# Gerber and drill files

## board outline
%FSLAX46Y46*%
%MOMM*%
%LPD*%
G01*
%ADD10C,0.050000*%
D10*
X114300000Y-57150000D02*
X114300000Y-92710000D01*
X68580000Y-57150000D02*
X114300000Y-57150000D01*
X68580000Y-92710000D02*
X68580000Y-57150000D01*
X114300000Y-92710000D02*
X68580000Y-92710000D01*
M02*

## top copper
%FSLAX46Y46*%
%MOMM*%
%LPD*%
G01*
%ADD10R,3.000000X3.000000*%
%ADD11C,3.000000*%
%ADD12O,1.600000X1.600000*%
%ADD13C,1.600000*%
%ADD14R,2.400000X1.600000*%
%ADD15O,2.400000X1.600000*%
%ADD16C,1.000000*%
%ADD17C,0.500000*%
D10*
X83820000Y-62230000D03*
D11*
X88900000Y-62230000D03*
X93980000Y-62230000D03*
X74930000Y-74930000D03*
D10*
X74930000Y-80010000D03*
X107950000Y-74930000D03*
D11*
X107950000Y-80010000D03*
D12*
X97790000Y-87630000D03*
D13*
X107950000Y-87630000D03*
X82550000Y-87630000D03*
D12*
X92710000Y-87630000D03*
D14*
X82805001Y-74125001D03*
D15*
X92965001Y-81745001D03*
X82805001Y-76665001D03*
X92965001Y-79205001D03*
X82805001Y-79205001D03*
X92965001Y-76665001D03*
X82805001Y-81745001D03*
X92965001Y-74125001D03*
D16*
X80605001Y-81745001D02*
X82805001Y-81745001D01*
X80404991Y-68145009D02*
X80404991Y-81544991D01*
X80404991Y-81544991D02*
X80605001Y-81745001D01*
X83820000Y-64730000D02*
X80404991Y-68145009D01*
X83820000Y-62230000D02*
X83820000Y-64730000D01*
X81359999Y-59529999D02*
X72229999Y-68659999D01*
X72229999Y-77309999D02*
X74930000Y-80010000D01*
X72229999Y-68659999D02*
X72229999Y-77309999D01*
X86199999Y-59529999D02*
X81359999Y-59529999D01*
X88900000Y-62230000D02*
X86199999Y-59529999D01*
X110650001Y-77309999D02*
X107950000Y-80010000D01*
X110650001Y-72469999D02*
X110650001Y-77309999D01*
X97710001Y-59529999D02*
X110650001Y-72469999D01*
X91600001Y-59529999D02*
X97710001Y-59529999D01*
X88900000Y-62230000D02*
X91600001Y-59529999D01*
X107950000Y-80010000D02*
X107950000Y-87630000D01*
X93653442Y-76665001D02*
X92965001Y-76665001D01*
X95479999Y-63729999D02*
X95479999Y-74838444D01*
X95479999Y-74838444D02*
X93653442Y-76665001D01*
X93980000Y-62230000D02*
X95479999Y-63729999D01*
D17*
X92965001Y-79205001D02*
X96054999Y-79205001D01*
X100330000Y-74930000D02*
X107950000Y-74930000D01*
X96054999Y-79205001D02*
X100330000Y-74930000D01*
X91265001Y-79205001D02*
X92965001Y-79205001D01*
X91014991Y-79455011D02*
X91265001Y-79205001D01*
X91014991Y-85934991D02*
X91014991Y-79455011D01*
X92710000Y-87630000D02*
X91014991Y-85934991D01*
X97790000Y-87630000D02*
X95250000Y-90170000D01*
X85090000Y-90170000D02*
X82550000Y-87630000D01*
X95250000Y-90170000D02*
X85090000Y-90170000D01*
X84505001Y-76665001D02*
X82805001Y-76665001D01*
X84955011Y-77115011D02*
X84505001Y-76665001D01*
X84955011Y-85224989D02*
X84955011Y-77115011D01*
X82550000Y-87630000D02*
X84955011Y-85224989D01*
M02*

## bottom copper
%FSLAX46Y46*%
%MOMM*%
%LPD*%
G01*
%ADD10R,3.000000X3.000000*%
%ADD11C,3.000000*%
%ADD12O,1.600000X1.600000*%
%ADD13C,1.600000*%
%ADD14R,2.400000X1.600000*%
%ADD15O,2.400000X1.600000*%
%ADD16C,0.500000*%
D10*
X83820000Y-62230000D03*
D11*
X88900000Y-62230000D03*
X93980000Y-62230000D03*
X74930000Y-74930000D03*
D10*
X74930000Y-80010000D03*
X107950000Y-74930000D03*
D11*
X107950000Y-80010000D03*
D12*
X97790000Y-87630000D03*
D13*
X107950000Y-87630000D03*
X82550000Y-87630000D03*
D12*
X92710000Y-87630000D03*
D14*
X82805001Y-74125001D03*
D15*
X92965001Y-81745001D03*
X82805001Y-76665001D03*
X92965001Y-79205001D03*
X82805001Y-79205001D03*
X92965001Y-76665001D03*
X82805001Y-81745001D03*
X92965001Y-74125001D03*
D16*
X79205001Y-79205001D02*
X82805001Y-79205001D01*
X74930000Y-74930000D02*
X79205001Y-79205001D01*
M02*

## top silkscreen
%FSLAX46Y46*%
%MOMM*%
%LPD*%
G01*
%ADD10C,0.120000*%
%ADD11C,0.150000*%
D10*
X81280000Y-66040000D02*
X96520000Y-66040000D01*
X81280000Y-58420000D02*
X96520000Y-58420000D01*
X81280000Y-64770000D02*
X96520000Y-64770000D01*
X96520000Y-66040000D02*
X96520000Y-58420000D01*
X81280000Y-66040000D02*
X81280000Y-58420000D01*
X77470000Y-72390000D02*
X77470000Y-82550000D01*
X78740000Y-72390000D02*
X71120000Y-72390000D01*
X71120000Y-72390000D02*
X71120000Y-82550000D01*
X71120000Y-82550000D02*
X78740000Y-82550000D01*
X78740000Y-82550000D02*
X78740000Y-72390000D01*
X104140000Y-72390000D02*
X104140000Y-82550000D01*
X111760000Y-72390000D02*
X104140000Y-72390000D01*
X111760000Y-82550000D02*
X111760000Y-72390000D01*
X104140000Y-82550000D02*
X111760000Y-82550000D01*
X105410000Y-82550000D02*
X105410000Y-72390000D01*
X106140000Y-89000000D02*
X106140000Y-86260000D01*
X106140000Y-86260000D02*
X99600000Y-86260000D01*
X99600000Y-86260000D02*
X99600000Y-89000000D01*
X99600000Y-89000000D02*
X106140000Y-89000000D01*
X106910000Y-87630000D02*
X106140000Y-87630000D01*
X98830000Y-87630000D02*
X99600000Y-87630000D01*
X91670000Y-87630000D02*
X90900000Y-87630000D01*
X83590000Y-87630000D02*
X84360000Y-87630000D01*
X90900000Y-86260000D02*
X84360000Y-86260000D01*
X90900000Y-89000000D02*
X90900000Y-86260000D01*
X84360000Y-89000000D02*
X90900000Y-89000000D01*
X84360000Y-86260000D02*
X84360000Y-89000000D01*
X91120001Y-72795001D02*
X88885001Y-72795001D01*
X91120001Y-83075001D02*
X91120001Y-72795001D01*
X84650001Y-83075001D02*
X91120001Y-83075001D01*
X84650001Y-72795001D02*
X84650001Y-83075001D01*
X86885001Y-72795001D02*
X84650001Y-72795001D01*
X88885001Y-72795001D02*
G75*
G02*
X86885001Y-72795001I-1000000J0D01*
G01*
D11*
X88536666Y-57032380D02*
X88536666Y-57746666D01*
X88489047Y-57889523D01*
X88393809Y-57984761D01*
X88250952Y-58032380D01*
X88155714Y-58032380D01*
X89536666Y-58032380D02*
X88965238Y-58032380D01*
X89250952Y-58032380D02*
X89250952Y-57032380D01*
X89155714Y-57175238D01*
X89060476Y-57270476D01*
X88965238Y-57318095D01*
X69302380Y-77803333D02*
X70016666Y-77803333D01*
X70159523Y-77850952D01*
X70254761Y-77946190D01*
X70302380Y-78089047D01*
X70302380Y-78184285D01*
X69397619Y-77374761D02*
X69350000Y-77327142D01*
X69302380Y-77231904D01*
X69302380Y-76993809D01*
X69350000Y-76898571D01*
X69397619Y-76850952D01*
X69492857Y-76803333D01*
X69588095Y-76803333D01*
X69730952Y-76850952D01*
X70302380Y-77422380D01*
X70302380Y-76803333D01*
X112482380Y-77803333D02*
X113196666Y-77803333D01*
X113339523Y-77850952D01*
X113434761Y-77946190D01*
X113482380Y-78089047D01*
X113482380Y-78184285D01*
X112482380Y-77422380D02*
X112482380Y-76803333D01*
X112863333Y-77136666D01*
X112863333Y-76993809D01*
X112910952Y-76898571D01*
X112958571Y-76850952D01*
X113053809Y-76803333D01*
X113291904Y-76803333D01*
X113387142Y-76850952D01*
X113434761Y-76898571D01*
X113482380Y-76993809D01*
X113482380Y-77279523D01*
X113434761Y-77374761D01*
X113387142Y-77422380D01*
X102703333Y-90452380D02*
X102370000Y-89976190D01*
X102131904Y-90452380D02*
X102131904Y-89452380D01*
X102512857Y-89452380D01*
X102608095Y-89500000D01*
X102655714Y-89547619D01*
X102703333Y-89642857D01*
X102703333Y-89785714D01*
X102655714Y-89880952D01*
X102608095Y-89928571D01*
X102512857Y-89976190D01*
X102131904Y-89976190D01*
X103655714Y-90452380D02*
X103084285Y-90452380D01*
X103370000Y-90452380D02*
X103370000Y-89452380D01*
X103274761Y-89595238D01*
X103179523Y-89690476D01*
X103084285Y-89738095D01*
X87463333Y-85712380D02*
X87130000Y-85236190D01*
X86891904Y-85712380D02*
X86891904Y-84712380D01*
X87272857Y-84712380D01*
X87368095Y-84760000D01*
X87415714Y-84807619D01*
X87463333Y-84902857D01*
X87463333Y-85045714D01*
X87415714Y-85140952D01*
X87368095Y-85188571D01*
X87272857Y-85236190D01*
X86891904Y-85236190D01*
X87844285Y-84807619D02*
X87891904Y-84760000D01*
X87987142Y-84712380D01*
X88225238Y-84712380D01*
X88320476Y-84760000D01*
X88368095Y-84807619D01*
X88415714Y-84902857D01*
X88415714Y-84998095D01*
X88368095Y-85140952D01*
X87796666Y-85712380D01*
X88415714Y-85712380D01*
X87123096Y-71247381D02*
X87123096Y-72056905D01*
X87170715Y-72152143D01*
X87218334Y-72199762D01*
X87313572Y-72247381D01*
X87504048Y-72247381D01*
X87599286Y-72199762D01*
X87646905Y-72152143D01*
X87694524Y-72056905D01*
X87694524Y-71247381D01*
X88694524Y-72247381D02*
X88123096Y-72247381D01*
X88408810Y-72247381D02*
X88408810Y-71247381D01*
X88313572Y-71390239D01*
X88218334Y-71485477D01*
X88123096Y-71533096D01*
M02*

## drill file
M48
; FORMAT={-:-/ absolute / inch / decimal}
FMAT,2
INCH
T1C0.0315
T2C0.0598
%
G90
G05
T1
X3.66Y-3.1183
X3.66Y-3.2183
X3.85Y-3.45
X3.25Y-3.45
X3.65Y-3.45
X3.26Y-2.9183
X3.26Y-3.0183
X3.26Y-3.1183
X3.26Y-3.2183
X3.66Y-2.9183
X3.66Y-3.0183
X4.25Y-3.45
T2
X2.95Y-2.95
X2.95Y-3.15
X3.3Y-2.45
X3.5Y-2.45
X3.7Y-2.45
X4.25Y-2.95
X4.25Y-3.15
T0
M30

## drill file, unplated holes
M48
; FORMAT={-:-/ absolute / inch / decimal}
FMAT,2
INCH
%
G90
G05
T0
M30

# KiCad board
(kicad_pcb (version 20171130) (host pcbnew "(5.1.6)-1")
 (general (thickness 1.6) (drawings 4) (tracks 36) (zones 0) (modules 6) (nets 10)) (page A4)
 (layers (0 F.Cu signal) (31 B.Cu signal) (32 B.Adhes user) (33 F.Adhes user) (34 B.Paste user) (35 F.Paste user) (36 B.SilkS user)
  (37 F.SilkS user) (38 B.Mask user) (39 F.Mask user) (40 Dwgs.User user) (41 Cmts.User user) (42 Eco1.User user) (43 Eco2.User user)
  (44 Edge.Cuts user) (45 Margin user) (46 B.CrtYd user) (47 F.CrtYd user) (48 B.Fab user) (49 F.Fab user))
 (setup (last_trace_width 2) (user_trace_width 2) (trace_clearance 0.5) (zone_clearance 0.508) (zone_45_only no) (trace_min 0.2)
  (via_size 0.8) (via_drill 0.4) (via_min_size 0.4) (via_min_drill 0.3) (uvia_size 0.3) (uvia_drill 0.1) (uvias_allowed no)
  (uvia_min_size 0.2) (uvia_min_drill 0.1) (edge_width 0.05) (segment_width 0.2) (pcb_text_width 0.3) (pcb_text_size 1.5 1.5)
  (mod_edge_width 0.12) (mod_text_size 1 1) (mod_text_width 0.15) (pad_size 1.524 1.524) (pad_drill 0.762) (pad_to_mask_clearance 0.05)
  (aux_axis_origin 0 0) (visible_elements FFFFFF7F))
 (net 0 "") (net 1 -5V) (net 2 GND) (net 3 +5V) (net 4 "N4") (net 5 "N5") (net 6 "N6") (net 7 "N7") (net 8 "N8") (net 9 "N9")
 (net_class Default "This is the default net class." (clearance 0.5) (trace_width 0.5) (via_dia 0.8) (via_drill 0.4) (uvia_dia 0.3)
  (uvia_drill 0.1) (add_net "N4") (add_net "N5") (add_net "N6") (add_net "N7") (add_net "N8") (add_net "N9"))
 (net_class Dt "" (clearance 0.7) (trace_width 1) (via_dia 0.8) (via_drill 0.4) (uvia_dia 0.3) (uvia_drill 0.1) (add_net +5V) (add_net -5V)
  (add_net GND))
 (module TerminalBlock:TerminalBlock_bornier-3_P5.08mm (layer F.Cu) (at 83.82 62.23)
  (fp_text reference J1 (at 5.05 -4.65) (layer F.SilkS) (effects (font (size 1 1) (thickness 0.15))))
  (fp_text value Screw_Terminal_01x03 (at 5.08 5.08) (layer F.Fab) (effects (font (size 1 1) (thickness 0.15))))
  (fp_line (start -2.54 3.81) (end 12.7 3.81) (layer F.SilkS) (width 0.12))
  (fp_line (start -2.54 -3.81) (end 12.7 -3.81) (layer F.SilkS) (width 0.12))
  (fp_line (start -2.54 2.54) (end 12.7 2.54) (layer F.SilkS) (width 0.12))
  (fp_line (start 12.7 3.81) (end 12.7 -3.81) (layer F.SilkS) (width 0.12))
  (fp_line (start -2.54 3.81) (end -2.54 -3.81) (layer F.SilkS) (width 0.12))
  (pad 1 thru_hole rect (at 0 0) (size 3 3) (drill 1.52) (layers *.Cu *.Mask) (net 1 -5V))
  (pad 2 thru_hole circle (at 5.08 0) (size 3 3) (drill 1.52) (layers *.Cu *.Mask) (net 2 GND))
  (pad 3 thru_hole circle (at 10.16 0) (size 3 3) (drill 1.52) (layers *.Cu *.Mask) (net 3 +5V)))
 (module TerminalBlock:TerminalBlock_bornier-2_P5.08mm (layer F.Cu) (at 74.93 80.01 90)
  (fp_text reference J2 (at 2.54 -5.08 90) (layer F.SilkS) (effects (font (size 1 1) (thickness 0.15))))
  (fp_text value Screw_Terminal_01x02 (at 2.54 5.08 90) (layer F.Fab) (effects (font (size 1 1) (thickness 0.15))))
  (fp_line (start 7.62 2.54) (end -2.54 2.54) (layer F.SilkS) (width 0.12))
  (fp_line (start 7.62 3.81) (end 7.62 -3.81) (layer F.SilkS) (width 0.12))
  (fp_line (start 7.62 -3.81) (end -2.54 -3.81) (layer F.SilkS) (width 0.12))
  (fp_line (start -2.54 -3.81) (end -2.54 3.81) (layer F.SilkS) (width 0.12))
  (fp_line (start -2.54 3.81) (end 7.62 3.81) (layer F.SilkS) (width 0.12))
  (pad 2 thru_hole circle (at 5.08 0 90) (size 3 3) (drill 1.52) (layers *.Cu *.Mask) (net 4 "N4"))
  (pad 1 thru_hole rect (at 0 0 90) (size 3 3) (drill 1.52) (layers *.Cu *.Mask) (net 2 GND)))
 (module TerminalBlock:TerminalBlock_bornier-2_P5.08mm (layer F.Cu) (at 107.95 74.93 270)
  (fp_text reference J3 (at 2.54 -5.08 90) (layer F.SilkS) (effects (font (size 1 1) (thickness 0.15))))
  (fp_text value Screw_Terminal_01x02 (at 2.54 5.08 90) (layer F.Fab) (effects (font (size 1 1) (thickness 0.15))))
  (fp_line (start -2.54 3.81) (end 7.62 3.81) (layer F.SilkS) (width 0.12))
  (fp_line (start -2.54 -3.81) (end -2.54 3.81) (layer F.SilkS) (width 0.12))
  (fp_line (start 7.62 -3.81) (end -2.54 -3.81) (layer F.SilkS) (width 0.12))
  (fp_line (start 7.62 3.81) (end 7.62 -3.81) (layer F.SilkS) (width 0.12))
  (fp_line (start 7.62 2.54) (end -2.54 2.54) (layer F.SilkS) (width 0.12))
  (pad 1 thru_hole rect (at 0 0 270) (size 3 3) (drill 1.52) (layers *.Cu *.Mask) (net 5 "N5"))
  (pad 2 thru_hole circle (at 5.08 0 270) (size 3 3) (drill 1.52) (layers *.Cu *.Mask) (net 2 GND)))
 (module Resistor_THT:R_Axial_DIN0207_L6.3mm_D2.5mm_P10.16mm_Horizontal (layer F.Cu) (at 107.95 87.63 180)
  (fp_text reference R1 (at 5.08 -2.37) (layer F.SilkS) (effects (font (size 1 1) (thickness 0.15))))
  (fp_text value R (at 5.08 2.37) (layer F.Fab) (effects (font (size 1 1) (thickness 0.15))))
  (fp_line (start 1.81 -1.37) (end 1.81 1.37) (layer F.SilkS) (width 0.12))
  (fp_line (start 1.81 1.37) (end 8.35 1.37) (layer F.SilkS) (width 0.12))
  (fp_line (start 8.35 1.37) (end 8.35 -1.37) (layer F.SilkS) (width 0.12))
  (fp_line (start 8.35 -1.37) (end 1.81 -1.37) (layer F.SilkS) (width 0.12))
  (fp_line (start 1.04 0) (end 1.81 0) (layer F.SilkS) (width 0.12))
  (fp_line (start 9.12 0) (end 8.35 0) (layer F.SilkS) (width 0.12))
  (pad 2 thru_hole oval (at 10.16 0 180) (size 1.6 1.6) (drill 0.8) (layers *.Cu *.Mask) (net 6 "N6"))
  (pad 1 thru_hole circle (at 0 0 180) (size 1.6 1.6) (drill 0.8) (layers *.Cu *.Mask) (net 2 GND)))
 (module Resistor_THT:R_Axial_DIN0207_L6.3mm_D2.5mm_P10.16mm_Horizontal (layer F.Cu) (at 82.55 87.63)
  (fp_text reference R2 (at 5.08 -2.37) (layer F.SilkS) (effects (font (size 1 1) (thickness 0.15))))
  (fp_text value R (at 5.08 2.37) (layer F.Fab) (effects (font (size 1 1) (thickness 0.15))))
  (fp_line (start 9.12 0) (end 8.35 0) (layer F.SilkS) (width 0.12))
  (fp_line (start 1.04 0) (end 1.81 0) (layer F.SilkS) (width 0.12))
  (fp_line (start 8.35 -1.37) (end 1.81 -1.37) (layer F.SilkS) (width 0.12))
  (fp_line (start 8.35 1.37) (end 8.35 -1.37) (layer F.SilkS) (width 0.12))
  (fp_line (start 1.81 1.37) (end 8.35 1.37) (layer F.SilkS) (width 0.12))
  (fp_line (start 1.81 -1.37) (end 1.81 1.37) (layer F.SilkS) (width 0.12))
  (pad 1 thru_hole circle (at 0 0) (size 1.6 1.6) (drill 0.8) (layers *.Cu *.Mask) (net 6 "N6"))
  (pad 2 thru_hole oval (at 10.16 0) (size 1.6 1.6) (drill 0.8) (layers *.Cu *.Mask) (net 5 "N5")))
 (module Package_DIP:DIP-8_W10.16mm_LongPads (layer F.Cu) (at 82.805001 74.125001)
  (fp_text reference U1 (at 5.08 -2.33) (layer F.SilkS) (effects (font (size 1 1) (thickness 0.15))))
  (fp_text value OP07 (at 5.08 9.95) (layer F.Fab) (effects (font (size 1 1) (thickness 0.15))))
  (fp_line (start 8.315 -1.33) (end 6.08 -1.33) (layer F.SilkS) (width 0.12))
  (fp_line (start 8.315 8.95) (end 8.315 -1.33) (layer F.SilkS) (width 0.12))
  (fp_line (start 1.845 8.95) (end 8.315 8.95) (layer F.SilkS) (width 0.12))
  (fp_line (start 1.845 -1.33) (end 1.845 8.95) (layer F.SilkS) (width 0.12))
  (fp_line (start 4.08 -1.33) (end 1.845 -1.33) (layer F.SilkS) (width 0.12))
  (fp_arc (start 5.08 -1.33) (end 4.08 -1.33) (angle -180) (layer F.SilkS) (width 0.12))
  (pad 1 thru_hole rect (at 0 0) (size 2.4 1.6) (drill 0.8) (layers *.Cu *.Mask) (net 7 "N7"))
  (pad 5 thru_hole oval (at 10.16 7.62) (size 2.4 1.6) (drill 0.8) (layers *.Cu *.Mask) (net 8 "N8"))
  (pad 2 thru_hole oval (at 0 2.54) (size 2.4 1.6) (drill 0.8) (layers *.Cu *.Mask) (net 6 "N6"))
  (pad 6 thru_hole oval (at 10.16 5.08) (size 2.4 1.6) (drill 0.8) (layers *.Cu *.Mask) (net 5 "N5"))
  (pad 3 thru_hole oval (at 0 5.08) (size 2.4 1.6) (drill 0.8) (layers *.Cu *.Mask) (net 4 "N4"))
  (pad 7 thru_hole oval (at 10.16 2.54) (size 2.4 1.6) (drill 0.8) (layers *.Cu *.Mask) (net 3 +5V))
  (pad 4 thru_hole oval (at 0 7.62) (size 2.4 1.6) (drill 0.8) (layers *.Cu *.Mask) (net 1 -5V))
  (pad 8 thru_hole oval (at 10.16 0) (size 2.4 1.6) (drill 0.8) (layers *.Cu *.Mask) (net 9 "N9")))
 (gr_line (start 114.3 57.15) (end 114.3 92.71) (layer Edge.Cuts) (width 0.05))
 (gr_line (start 68.58 57.15) (end 114.3 57.15) (layer Edge.Cuts) (width 0.05))
 (gr_line (start 68.58 92.71) (end 68.58 57.15) (layer Edge.Cuts) (width 0.05))
 (gr_line (start 114.3 92.71) (end 68.58 92.71) (layer Edge.Cuts) (width 0.05))
 (segment (start 80.605001 81.745001) (end 82.805001 81.745001) (width 1) (layer F.Cu) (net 1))
 (segment (start 80.404991 68.145009) (end 80.404991 81.544991) (width 1) (layer F.Cu) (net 1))
 (segment (start 80.404991 81.544991) (end 80.605001 81.745001) (width 1) (layer F.Cu) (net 1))
 (segment (start 83.82 64.73) (end 80.404991 68.145009) (width 1) (layer F.Cu) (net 1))
 (segment (start 83.82 62.23) (end 83.82 64.73) (width 1) (layer F.Cu) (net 1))
 (segment (start 81.359999 59.529999) (end 72.229999 68.659999) (width 1) (layer F.Cu) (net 2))
 (segment (start 72.229999 77.309999) (end 74.93 80.01) (width 1) (layer F.Cu) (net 2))
 (segment (start 72.229999 68.659999) (end 72.229999 77.309999) (width 1) (layer F.Cu) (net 2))
 (segment (start 86.199999 59.529999) (end 81.359999 59.529999) (width 1) (layer F.Cu) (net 2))
 (segment (start 88.9 62.23) (end 86.199999 59.529999) (width 1) (layer F.Cu) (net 2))
 (segment (start 110.650001 77.309999) (end 107.95 80.01) (width 1) (layer F.Cu) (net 2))
 (segment (start 110.650001 72.469999) (end 110.650001 77.309999) (width 1) (layer F.Cu) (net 2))
 (segment (start 97.710001 59.529999) (end 110.650001 72.469999) (width 1) (layer F.Cu) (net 2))
 (segment (start 91.600001 59.529999) (end 97.710001 59.529999) (width 1) (layer F.Cu) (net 2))
 (segment (start 88.9 62.23) (end 91.600001 59.529999) (width 1) (layer F.Cu) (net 2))
 (segment (start 107.95 80.01) (end 107.95 87.63) (width 1) (layer F.Cu) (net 2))
 (segment (start 93.653442 76.665001) (end 92.965001 76.665001) (width 1) (layer F.Cu) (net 3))
 (segment (start 95.479999 63.729999) (end 95.479999 74.838444) (width 1) (layer F.Cu) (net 3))
 (segment (start 95.479999 74.838444) (end 93.653442 76.665001) (width 1) (layer F.Cu) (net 3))
 (segment (start 93.98 62.23) (end 95.479999 63.729999) (width 1) (layer F.Cu) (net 3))
 (segment (start 79.205001 79.205001) (end 82.805001 79.205001) (width 0.5) (layer B.Cu) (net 4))
 (segment (start 74.93 74.93) (end 79.205001 79.205001) (width 0.5) (layer B.Cu) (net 4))
 (segment (start 92.965001 79.205001) (end 96.054999 79.205001) (width 0.5) (layer F.Cu) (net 5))
 (segment (start 100.33 74.93) (end 107.95 74.93) (width 0.5) (layer F.Cu) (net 5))
 (segment (start 96.054999 79.205001) (end 100.33 74.93) (width 0.5) (layer F.Cu) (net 5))
 (segment (start 91.265001 79.205001) (end 92.965001 79.205001) (width 0.5) (layer F.Cu) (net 5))
 (segment (start 91.014991 79.455011) (end 91.265001 79.205001) (width 0.5) (layer F.Cu) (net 5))
 (segment (start 91.014991 85.934991) (end 91.014991 79.455011) (width 0.5) (layer F.Cu) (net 5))
 (segment (start 92.71 87.63) (end 91.014991 85.934991) (width 0.5) (layer F.Cu) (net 5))
 (segment (start 97.79 87.63) (end 95.25 90.17) (width 0.5) (layer F.Cu) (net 6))
 (segment (start 85.09 90.17) (end 82.55 87.63) (width 0.5) (layer F.Cu) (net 6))
 (segment (start 95.25 90.17) (end 85.09 90.17) (width 0.5) (layer F.Cu) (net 6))
 (segment (start 84.505001 76.665001) (end 82.805001 76.665001) (width 0.5) (layer F.Cu) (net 6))
 (segment (start 84.955011 77.115011) (end 84.505001 76.665001) (width 0.5) (layer F.Cu) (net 6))
 (segment (start 84.955011 85.224989) (end 84.955011 77.115011) (width 0.5) (layer F.Cu) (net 6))
 (segment (start 82.55 87.63) (end 84.955011 85.224989) (width 0.5) (layer F.Cu) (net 6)))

